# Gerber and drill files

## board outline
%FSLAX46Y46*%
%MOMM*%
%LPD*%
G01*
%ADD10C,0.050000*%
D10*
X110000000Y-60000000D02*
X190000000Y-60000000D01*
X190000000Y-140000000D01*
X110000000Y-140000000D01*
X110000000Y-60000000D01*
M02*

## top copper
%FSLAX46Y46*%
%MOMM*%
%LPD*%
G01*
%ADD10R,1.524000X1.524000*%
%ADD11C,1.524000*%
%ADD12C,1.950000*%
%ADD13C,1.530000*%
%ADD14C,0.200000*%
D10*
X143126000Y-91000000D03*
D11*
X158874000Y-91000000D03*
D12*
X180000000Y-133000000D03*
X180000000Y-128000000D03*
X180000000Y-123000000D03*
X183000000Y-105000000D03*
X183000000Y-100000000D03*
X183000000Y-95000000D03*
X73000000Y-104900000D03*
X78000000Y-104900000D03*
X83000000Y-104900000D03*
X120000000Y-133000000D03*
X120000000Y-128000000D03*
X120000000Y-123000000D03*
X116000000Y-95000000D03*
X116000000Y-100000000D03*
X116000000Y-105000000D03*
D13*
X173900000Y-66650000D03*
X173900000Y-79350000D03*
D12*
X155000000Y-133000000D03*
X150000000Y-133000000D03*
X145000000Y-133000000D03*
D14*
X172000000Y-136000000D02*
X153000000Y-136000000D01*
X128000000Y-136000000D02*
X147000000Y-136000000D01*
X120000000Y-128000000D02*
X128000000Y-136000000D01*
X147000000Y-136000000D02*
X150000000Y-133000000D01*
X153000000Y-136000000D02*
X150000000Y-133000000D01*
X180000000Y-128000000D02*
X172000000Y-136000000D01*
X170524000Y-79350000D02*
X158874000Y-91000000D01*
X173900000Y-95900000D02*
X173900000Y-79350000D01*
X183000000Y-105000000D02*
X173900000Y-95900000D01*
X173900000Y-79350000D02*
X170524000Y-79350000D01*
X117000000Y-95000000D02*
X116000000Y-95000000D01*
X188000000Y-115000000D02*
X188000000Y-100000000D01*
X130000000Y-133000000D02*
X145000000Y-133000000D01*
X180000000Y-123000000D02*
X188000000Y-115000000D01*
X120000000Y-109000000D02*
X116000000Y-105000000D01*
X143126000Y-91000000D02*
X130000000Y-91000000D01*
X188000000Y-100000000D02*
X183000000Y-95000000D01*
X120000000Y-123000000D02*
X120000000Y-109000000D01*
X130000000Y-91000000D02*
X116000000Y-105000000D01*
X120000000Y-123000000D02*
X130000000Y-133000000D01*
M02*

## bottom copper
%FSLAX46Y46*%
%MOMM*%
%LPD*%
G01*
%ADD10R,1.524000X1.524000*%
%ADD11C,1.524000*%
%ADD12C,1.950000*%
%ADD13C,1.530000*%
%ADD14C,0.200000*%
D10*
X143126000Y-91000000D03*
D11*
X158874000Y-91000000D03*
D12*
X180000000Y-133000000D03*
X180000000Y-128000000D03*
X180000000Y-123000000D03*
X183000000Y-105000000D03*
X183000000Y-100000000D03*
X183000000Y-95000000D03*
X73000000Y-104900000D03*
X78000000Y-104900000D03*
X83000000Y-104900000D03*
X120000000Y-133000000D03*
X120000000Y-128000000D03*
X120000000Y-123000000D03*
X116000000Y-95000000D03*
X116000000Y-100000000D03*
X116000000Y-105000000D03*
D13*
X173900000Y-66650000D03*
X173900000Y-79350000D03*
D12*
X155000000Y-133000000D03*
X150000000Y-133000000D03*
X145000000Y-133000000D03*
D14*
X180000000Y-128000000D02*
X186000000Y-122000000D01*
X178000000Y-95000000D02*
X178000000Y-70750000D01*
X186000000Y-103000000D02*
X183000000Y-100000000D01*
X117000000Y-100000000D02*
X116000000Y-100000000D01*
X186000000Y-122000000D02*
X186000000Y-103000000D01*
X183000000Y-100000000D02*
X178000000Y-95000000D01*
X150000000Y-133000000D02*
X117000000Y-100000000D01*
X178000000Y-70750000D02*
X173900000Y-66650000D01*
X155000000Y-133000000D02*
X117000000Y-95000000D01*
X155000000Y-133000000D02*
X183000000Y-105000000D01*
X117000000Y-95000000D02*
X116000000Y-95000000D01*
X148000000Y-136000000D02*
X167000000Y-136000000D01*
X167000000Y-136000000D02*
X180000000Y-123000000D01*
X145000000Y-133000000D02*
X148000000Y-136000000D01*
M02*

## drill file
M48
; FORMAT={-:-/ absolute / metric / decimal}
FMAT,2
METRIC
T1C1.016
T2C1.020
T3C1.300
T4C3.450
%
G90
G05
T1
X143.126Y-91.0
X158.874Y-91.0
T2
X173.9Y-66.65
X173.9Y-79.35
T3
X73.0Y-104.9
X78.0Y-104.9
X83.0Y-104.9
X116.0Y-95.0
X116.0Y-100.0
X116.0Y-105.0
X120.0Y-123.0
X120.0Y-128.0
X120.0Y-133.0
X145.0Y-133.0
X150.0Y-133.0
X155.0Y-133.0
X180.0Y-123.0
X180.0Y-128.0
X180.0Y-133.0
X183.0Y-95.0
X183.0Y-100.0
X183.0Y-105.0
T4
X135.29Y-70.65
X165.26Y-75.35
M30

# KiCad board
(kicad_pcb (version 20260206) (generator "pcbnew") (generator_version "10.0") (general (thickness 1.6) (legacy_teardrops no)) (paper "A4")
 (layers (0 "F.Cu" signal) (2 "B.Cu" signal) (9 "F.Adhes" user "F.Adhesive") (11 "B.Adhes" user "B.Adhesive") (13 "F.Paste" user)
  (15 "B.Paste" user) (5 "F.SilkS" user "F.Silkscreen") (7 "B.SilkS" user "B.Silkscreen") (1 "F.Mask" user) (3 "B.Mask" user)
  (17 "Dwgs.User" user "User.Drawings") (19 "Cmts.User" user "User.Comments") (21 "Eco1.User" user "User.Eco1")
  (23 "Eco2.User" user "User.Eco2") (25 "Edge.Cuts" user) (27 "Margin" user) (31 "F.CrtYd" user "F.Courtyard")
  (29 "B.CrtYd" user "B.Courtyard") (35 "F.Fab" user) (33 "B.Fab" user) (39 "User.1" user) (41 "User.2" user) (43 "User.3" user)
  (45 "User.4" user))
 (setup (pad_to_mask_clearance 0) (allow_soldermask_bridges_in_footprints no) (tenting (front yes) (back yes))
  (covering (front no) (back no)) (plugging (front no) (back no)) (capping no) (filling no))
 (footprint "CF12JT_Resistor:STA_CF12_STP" (layer "F.Cu") (at 143.126 91)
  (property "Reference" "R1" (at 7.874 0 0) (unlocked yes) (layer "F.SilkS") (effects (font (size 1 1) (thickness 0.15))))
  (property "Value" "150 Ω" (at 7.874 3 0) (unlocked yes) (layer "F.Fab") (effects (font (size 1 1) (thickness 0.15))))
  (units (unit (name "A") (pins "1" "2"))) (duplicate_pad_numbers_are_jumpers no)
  (pad "1" thru_hole rect (at 0 0) (size 1.524 1.524) (drill 1.016) (layers "*.Cu" "*.Mask") (remove_unused_layers no) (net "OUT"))
  (pad "2" thru_hole circle (at 15.748 0) (size 1.524 1.524) (drill 1.016) (layers "*.Cu" "*.Mask") (remove_unused_layers no) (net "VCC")))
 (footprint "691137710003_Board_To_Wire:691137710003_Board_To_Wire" (layer "F.Cu") (at 180 128 90)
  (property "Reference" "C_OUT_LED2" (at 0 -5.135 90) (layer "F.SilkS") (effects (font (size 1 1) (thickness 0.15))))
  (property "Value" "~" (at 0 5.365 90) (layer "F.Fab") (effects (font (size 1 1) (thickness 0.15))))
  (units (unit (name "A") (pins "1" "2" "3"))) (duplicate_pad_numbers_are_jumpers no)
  (pad "1" thru_hole circle (at -5 0 90) (size 1.95 1.95) (drill 1.3) (layers "*.Cu" "*.Mask") (remove_unused_layers no)
   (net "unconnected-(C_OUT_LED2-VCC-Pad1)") (solder_mask_margin 0.102))
  (pad "2" thru_hole circle (at 0 0 90) (size 1.95 1.95) (drill 1.3) (layers "*.Cu" "*.Mask") (remove_unused_layers no) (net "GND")
   (solder_mask_margin 0.102))
  (pad "3" thru_hole circle (at 5 0 90) (size 1.95 1.95) (drill 1.3) (layers "*.Cu" "*.Mask") (remove_unused_layers no) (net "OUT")
   (solder_mask_margin 0.102)))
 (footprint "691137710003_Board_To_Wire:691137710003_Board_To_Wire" (layer "F.Cu") (at 183 100 90)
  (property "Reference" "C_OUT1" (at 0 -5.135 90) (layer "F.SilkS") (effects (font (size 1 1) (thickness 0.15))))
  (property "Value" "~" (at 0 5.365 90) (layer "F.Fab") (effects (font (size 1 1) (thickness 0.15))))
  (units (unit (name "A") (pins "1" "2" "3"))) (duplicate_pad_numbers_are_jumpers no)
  (pad "1" thru_hole circle (at -5 0 90) (size 1.95 1.95) (drill 1.3) (layers "*.Cu" "*.Mask") (remove_unused_layers no) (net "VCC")
   (solder_mask_margin 0.102))
  (pad "2" thru_hole circle (at 0 0 90) (size 1.95 1.95) (drill 1.3) (layers "*.Cu" "*.Mask") (remove_unused_layers no) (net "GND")
   (solder_mask_margin 0.102))
  (pad "3" thru_hole circle (at 5 0 90) (size 1.95 1.95) (drill 1.3) (layers "*.Cu" "*.Mask") (remove_unused_layers no) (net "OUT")
   (solder_mask_margin 0.102)))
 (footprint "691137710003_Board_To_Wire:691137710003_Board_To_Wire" (layer "F.Cu") (at 78 104.9)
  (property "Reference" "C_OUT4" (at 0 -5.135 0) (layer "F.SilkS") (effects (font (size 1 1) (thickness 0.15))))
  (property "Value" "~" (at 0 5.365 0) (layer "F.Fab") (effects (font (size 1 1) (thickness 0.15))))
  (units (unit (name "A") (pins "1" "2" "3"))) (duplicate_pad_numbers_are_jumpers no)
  (pad "1" thru_hole circle (at -5 0) (size 1.95 1.95) (drill 1.3) (layers "*.Cu" "*.Mask") (remove_unused_layers no) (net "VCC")
   (solder_mask_margin 0.102))
  (pad "2" thru_hole circle (at 0 0) (size 1.95 1.95) (drill 1.3) (layers "*.Cu" "*.Mask") (remove_unused_layers no) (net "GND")
   (solder_mask_margin 0.102))
  (pad "3" thru_hole circle (at 5 0) (size 1.95 1.95) (drill 1.3) (layers "*.Cu" "*.Mask") (remove_unused_layers no) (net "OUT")
   (solder_mask_margin 0.102)))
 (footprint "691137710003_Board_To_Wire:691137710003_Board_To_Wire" (layer "F.Cu") (at 120 128 90)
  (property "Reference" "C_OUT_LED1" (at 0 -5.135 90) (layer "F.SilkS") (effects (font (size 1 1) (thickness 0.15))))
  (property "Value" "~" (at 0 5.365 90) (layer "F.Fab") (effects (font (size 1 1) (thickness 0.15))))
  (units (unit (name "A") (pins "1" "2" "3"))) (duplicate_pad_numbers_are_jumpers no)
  (pad "1" thru_hole circle (at -5 0 90) (size 1.95 1.95) (drill 1.3) (layers "*.Cu" "*.Mask") (remove_unused_layers no)
   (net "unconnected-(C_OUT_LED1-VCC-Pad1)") (solder_mask_margin 0.102))
  (pad "2" thru_hole circle (at 0 0 90) (size 1.95 1.95) (drill 1.3) (layers "*.Cu" "*.Mask") (remove_unused_layers no) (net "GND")
   (solder_mask_margin 0.102))
  (pad "3" thru_hole circle (at 5 0 90) (size 1.95 1.95) (drill 1.3) (layers "*.Cu" "*.Mask") (remove_unused_layers no) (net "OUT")
   (solder_mask_margin 0.102)))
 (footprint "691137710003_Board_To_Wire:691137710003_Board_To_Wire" (layer "F.Cu") (at 116 100 -90)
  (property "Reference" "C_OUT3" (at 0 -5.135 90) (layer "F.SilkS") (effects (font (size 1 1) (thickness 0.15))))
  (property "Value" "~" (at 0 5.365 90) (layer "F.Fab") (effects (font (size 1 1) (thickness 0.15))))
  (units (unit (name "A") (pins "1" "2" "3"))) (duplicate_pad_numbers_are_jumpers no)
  (pad "1" thru_hole circle (at -5 0 270) (size 1.95 1.95) (drill 1.3) (layers "*.Cu" "*.Mask") (remove_unused_layers no) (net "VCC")
   (solder_mask_margin 0.102))
  (pad "2" thru_hole circle (at 0 0 270) (size 1.95 1.95) (drill 1.3) (layers "*.Cu" "*.Mask") (remove_unused_layers no) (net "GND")
   (solder_mask_margin 0.102))
  (pad "3" thru_hole circle (at 5 0 270) (size 1.95 1.95) (drill 1.3) (layers "*.Cu" "*.Mask") (remove_unused_layers no) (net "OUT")
   (solder_mask_margin 0.102)))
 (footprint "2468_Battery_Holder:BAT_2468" (layer "F.Cu") (at 150 73)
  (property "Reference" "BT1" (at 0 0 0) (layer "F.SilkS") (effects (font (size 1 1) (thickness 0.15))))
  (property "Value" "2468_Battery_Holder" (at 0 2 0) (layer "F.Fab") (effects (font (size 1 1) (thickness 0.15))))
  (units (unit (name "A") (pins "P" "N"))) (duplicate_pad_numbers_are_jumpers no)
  (pad "" np_thru_hole circle (at -14.71 -2.35) (size 3.45 3.45) (drill 3.45) (layers "*.Cu" "*.Mask"))
  (pad "" np_thru_hole circle (at 15.26 2.35) (size 3.45 3.45) (drill 3.45) (layers "*.Cu" "*.Mask"))
  (pad "N" thru_hole circle (at 23.9 -6.35) (size 1.53 1.53) (drill 1.02) (layers "*.Cu" "*.Mask") (remove_unused_layers no) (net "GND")
   (solder_mask_margin 0.102))
  (pad "P" thru_hole circle (at 23.9 6.35) (size 1.53 1.53) (drill 1.02) (layers "*.Cu" "*.Mask") (remove_unused_layers no) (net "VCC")
   (solder_mask_margin 0.102)))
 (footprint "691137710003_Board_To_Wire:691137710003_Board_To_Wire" (layer "F.Cu") (at 150 133 180)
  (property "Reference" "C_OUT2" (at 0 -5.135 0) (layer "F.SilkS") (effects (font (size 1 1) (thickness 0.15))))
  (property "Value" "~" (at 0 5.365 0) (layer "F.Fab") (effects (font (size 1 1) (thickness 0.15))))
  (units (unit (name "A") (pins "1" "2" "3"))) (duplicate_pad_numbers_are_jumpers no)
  (pad "1" thru_hole circle (at -5 0 180) (size 1.95 1.95) (drill 1.3) (layers "*.Cu" "*.Mask") (remove_unused_layers no) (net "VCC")
   (solder_mask_margin 0.102))
  (pad "2" thru_hole circle (at 0 0 180) (size 1.95 1.95) (drill 1.3) (layers "*.Cu" "*.Mask") (remove_unused_layers no) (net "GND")
   (solder_mask_margin 0.102))
  (pad "3" thru_hole circle (at 5 0 180) (size 1.95 1.95) (drill 1.3) (layers "*.Cu" "*.Mask") (remove_unused_layers no) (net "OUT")
   (solder_mask_margin 0.102)))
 (gr_rect (start 110 60) (end 190 140) (stroke (width 0.05) (type solid)) (fill no) (layer "Edge.Cuts"))
 (segment (start 172 136) (end 153 136) (width 0.2) (layer "F.Cu") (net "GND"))
 (segment (start 128 136) (end 147 136) (width 0.2) (layer "F.Cu") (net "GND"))
 (segment (start 120 128) (end 128 136) (width 0.2) (layer "F.Cu") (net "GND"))
 (segment (start 147 136) (end 150 133) (width 0.2) (layer "F.Cu") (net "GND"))
 (segment (start 153 136) (end 150 133) (width 0.2) (layer "F.Cu") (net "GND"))
 (segment (start 180 128) (end 172 136) (width 0.2) (layer "F.Cu") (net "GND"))
 (segment (start 180 128) (end 186 122) (width 0.2) (layer "B.Cu") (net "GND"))
 (segment (start 178 95) (end 178 70.75) (width 0.2) (layer "B.Cu") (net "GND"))
 (segment (start 186 103) (end 183 100) (width 0.2) (layer "B.Cu") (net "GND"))
 (segment (start 117 100) (end 116 100) (width 0.2) (layer "B.Cu") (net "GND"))
 (segment (start 186 122) (end 186 103) (width 0.2) (layer "B.Cu") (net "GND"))
 (segment (start 183 100) (end 178 95) (width 0.2) (layer "B.Cu") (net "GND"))
 (segment (start 150 133) (end 117 100) (width 0.2) (layer "B.Cu") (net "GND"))
 (segment (start 178 70.75) (end 173.9 66.65) (width 0.2) (layer "B.Cu") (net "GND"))
 (segment (start 170.524 79.35) (end 158.874 91) (width 0.2) (layer "F.Cu") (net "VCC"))
 (segment (start 173.9 95.9) (end 173.9 79.35) (width 0.2) (layer "F.Cu") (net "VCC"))
 (segment (start 183 105) (end 173.9 95.9) (width 0.2) (layer "F.Cu") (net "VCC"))
 (segment (start 173.9 79.35) (end 170.524 79.35) (width 0.2) (layer "F.Cu") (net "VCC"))
 (segment (start 117 95) (end 116 95) (width 0.2) (layer "F.Cu") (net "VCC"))
 (segment (start 155 133) (end 117 95) (width 0.2) (layer "B.Cu") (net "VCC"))
 (segment (start 155 133) (end 183 105) (width 0.2) (layer "B.Cu") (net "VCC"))
 (segment (start 117 95) (end 116 95) (width 0.2) (layer "B.Cu") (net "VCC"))
 (segment (start 188 115) (end 188 100) (width 0.2) (layer "F.Cu") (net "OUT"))
 (segment (start 130 133) (end 145 133) (width 0.2) (layer "F.Cu") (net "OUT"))
 (segment (start 180 123) (end 188 115) (width 0.2) (layer "F.Cu") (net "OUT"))
 (segment (start 120 109) (end 116 105) (width 0.2) (layer "F.Cu") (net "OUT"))
 (segment (start 143.126 91) (end 130 91) (width 0.2) (layer "F.Cu") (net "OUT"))
 (segment (start 188 100) (end 183 95) (width 0.2) (layer "F.Cu") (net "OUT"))
 (segment (start 120 123) (end 120 109) (width 0.2) (layer "F.Cu") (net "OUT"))
 (segment (start 130 91) (end 116 105) (width 0.2) (layer "F.Cu") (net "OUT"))
 (segment (start 120 123) (end 130 133) (width 0.2) (layer "F.Cu") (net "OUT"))
 (segment (start 148 136) (end 167 136) (width 0.2) (layer "B.Cu") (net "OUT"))
 (segment (start 167 136) (end 180 123) (width 0.2) (layer "B.Cu") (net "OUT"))
 (segment (start 145 133) (end 148 136) (width 0.2) (layer "B.Cu") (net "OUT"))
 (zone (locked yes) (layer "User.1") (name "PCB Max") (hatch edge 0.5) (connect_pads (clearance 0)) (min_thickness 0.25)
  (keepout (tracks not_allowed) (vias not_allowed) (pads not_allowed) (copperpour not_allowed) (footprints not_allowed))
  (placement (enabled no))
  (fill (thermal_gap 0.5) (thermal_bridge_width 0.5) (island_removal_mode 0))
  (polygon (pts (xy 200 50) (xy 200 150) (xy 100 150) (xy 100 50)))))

